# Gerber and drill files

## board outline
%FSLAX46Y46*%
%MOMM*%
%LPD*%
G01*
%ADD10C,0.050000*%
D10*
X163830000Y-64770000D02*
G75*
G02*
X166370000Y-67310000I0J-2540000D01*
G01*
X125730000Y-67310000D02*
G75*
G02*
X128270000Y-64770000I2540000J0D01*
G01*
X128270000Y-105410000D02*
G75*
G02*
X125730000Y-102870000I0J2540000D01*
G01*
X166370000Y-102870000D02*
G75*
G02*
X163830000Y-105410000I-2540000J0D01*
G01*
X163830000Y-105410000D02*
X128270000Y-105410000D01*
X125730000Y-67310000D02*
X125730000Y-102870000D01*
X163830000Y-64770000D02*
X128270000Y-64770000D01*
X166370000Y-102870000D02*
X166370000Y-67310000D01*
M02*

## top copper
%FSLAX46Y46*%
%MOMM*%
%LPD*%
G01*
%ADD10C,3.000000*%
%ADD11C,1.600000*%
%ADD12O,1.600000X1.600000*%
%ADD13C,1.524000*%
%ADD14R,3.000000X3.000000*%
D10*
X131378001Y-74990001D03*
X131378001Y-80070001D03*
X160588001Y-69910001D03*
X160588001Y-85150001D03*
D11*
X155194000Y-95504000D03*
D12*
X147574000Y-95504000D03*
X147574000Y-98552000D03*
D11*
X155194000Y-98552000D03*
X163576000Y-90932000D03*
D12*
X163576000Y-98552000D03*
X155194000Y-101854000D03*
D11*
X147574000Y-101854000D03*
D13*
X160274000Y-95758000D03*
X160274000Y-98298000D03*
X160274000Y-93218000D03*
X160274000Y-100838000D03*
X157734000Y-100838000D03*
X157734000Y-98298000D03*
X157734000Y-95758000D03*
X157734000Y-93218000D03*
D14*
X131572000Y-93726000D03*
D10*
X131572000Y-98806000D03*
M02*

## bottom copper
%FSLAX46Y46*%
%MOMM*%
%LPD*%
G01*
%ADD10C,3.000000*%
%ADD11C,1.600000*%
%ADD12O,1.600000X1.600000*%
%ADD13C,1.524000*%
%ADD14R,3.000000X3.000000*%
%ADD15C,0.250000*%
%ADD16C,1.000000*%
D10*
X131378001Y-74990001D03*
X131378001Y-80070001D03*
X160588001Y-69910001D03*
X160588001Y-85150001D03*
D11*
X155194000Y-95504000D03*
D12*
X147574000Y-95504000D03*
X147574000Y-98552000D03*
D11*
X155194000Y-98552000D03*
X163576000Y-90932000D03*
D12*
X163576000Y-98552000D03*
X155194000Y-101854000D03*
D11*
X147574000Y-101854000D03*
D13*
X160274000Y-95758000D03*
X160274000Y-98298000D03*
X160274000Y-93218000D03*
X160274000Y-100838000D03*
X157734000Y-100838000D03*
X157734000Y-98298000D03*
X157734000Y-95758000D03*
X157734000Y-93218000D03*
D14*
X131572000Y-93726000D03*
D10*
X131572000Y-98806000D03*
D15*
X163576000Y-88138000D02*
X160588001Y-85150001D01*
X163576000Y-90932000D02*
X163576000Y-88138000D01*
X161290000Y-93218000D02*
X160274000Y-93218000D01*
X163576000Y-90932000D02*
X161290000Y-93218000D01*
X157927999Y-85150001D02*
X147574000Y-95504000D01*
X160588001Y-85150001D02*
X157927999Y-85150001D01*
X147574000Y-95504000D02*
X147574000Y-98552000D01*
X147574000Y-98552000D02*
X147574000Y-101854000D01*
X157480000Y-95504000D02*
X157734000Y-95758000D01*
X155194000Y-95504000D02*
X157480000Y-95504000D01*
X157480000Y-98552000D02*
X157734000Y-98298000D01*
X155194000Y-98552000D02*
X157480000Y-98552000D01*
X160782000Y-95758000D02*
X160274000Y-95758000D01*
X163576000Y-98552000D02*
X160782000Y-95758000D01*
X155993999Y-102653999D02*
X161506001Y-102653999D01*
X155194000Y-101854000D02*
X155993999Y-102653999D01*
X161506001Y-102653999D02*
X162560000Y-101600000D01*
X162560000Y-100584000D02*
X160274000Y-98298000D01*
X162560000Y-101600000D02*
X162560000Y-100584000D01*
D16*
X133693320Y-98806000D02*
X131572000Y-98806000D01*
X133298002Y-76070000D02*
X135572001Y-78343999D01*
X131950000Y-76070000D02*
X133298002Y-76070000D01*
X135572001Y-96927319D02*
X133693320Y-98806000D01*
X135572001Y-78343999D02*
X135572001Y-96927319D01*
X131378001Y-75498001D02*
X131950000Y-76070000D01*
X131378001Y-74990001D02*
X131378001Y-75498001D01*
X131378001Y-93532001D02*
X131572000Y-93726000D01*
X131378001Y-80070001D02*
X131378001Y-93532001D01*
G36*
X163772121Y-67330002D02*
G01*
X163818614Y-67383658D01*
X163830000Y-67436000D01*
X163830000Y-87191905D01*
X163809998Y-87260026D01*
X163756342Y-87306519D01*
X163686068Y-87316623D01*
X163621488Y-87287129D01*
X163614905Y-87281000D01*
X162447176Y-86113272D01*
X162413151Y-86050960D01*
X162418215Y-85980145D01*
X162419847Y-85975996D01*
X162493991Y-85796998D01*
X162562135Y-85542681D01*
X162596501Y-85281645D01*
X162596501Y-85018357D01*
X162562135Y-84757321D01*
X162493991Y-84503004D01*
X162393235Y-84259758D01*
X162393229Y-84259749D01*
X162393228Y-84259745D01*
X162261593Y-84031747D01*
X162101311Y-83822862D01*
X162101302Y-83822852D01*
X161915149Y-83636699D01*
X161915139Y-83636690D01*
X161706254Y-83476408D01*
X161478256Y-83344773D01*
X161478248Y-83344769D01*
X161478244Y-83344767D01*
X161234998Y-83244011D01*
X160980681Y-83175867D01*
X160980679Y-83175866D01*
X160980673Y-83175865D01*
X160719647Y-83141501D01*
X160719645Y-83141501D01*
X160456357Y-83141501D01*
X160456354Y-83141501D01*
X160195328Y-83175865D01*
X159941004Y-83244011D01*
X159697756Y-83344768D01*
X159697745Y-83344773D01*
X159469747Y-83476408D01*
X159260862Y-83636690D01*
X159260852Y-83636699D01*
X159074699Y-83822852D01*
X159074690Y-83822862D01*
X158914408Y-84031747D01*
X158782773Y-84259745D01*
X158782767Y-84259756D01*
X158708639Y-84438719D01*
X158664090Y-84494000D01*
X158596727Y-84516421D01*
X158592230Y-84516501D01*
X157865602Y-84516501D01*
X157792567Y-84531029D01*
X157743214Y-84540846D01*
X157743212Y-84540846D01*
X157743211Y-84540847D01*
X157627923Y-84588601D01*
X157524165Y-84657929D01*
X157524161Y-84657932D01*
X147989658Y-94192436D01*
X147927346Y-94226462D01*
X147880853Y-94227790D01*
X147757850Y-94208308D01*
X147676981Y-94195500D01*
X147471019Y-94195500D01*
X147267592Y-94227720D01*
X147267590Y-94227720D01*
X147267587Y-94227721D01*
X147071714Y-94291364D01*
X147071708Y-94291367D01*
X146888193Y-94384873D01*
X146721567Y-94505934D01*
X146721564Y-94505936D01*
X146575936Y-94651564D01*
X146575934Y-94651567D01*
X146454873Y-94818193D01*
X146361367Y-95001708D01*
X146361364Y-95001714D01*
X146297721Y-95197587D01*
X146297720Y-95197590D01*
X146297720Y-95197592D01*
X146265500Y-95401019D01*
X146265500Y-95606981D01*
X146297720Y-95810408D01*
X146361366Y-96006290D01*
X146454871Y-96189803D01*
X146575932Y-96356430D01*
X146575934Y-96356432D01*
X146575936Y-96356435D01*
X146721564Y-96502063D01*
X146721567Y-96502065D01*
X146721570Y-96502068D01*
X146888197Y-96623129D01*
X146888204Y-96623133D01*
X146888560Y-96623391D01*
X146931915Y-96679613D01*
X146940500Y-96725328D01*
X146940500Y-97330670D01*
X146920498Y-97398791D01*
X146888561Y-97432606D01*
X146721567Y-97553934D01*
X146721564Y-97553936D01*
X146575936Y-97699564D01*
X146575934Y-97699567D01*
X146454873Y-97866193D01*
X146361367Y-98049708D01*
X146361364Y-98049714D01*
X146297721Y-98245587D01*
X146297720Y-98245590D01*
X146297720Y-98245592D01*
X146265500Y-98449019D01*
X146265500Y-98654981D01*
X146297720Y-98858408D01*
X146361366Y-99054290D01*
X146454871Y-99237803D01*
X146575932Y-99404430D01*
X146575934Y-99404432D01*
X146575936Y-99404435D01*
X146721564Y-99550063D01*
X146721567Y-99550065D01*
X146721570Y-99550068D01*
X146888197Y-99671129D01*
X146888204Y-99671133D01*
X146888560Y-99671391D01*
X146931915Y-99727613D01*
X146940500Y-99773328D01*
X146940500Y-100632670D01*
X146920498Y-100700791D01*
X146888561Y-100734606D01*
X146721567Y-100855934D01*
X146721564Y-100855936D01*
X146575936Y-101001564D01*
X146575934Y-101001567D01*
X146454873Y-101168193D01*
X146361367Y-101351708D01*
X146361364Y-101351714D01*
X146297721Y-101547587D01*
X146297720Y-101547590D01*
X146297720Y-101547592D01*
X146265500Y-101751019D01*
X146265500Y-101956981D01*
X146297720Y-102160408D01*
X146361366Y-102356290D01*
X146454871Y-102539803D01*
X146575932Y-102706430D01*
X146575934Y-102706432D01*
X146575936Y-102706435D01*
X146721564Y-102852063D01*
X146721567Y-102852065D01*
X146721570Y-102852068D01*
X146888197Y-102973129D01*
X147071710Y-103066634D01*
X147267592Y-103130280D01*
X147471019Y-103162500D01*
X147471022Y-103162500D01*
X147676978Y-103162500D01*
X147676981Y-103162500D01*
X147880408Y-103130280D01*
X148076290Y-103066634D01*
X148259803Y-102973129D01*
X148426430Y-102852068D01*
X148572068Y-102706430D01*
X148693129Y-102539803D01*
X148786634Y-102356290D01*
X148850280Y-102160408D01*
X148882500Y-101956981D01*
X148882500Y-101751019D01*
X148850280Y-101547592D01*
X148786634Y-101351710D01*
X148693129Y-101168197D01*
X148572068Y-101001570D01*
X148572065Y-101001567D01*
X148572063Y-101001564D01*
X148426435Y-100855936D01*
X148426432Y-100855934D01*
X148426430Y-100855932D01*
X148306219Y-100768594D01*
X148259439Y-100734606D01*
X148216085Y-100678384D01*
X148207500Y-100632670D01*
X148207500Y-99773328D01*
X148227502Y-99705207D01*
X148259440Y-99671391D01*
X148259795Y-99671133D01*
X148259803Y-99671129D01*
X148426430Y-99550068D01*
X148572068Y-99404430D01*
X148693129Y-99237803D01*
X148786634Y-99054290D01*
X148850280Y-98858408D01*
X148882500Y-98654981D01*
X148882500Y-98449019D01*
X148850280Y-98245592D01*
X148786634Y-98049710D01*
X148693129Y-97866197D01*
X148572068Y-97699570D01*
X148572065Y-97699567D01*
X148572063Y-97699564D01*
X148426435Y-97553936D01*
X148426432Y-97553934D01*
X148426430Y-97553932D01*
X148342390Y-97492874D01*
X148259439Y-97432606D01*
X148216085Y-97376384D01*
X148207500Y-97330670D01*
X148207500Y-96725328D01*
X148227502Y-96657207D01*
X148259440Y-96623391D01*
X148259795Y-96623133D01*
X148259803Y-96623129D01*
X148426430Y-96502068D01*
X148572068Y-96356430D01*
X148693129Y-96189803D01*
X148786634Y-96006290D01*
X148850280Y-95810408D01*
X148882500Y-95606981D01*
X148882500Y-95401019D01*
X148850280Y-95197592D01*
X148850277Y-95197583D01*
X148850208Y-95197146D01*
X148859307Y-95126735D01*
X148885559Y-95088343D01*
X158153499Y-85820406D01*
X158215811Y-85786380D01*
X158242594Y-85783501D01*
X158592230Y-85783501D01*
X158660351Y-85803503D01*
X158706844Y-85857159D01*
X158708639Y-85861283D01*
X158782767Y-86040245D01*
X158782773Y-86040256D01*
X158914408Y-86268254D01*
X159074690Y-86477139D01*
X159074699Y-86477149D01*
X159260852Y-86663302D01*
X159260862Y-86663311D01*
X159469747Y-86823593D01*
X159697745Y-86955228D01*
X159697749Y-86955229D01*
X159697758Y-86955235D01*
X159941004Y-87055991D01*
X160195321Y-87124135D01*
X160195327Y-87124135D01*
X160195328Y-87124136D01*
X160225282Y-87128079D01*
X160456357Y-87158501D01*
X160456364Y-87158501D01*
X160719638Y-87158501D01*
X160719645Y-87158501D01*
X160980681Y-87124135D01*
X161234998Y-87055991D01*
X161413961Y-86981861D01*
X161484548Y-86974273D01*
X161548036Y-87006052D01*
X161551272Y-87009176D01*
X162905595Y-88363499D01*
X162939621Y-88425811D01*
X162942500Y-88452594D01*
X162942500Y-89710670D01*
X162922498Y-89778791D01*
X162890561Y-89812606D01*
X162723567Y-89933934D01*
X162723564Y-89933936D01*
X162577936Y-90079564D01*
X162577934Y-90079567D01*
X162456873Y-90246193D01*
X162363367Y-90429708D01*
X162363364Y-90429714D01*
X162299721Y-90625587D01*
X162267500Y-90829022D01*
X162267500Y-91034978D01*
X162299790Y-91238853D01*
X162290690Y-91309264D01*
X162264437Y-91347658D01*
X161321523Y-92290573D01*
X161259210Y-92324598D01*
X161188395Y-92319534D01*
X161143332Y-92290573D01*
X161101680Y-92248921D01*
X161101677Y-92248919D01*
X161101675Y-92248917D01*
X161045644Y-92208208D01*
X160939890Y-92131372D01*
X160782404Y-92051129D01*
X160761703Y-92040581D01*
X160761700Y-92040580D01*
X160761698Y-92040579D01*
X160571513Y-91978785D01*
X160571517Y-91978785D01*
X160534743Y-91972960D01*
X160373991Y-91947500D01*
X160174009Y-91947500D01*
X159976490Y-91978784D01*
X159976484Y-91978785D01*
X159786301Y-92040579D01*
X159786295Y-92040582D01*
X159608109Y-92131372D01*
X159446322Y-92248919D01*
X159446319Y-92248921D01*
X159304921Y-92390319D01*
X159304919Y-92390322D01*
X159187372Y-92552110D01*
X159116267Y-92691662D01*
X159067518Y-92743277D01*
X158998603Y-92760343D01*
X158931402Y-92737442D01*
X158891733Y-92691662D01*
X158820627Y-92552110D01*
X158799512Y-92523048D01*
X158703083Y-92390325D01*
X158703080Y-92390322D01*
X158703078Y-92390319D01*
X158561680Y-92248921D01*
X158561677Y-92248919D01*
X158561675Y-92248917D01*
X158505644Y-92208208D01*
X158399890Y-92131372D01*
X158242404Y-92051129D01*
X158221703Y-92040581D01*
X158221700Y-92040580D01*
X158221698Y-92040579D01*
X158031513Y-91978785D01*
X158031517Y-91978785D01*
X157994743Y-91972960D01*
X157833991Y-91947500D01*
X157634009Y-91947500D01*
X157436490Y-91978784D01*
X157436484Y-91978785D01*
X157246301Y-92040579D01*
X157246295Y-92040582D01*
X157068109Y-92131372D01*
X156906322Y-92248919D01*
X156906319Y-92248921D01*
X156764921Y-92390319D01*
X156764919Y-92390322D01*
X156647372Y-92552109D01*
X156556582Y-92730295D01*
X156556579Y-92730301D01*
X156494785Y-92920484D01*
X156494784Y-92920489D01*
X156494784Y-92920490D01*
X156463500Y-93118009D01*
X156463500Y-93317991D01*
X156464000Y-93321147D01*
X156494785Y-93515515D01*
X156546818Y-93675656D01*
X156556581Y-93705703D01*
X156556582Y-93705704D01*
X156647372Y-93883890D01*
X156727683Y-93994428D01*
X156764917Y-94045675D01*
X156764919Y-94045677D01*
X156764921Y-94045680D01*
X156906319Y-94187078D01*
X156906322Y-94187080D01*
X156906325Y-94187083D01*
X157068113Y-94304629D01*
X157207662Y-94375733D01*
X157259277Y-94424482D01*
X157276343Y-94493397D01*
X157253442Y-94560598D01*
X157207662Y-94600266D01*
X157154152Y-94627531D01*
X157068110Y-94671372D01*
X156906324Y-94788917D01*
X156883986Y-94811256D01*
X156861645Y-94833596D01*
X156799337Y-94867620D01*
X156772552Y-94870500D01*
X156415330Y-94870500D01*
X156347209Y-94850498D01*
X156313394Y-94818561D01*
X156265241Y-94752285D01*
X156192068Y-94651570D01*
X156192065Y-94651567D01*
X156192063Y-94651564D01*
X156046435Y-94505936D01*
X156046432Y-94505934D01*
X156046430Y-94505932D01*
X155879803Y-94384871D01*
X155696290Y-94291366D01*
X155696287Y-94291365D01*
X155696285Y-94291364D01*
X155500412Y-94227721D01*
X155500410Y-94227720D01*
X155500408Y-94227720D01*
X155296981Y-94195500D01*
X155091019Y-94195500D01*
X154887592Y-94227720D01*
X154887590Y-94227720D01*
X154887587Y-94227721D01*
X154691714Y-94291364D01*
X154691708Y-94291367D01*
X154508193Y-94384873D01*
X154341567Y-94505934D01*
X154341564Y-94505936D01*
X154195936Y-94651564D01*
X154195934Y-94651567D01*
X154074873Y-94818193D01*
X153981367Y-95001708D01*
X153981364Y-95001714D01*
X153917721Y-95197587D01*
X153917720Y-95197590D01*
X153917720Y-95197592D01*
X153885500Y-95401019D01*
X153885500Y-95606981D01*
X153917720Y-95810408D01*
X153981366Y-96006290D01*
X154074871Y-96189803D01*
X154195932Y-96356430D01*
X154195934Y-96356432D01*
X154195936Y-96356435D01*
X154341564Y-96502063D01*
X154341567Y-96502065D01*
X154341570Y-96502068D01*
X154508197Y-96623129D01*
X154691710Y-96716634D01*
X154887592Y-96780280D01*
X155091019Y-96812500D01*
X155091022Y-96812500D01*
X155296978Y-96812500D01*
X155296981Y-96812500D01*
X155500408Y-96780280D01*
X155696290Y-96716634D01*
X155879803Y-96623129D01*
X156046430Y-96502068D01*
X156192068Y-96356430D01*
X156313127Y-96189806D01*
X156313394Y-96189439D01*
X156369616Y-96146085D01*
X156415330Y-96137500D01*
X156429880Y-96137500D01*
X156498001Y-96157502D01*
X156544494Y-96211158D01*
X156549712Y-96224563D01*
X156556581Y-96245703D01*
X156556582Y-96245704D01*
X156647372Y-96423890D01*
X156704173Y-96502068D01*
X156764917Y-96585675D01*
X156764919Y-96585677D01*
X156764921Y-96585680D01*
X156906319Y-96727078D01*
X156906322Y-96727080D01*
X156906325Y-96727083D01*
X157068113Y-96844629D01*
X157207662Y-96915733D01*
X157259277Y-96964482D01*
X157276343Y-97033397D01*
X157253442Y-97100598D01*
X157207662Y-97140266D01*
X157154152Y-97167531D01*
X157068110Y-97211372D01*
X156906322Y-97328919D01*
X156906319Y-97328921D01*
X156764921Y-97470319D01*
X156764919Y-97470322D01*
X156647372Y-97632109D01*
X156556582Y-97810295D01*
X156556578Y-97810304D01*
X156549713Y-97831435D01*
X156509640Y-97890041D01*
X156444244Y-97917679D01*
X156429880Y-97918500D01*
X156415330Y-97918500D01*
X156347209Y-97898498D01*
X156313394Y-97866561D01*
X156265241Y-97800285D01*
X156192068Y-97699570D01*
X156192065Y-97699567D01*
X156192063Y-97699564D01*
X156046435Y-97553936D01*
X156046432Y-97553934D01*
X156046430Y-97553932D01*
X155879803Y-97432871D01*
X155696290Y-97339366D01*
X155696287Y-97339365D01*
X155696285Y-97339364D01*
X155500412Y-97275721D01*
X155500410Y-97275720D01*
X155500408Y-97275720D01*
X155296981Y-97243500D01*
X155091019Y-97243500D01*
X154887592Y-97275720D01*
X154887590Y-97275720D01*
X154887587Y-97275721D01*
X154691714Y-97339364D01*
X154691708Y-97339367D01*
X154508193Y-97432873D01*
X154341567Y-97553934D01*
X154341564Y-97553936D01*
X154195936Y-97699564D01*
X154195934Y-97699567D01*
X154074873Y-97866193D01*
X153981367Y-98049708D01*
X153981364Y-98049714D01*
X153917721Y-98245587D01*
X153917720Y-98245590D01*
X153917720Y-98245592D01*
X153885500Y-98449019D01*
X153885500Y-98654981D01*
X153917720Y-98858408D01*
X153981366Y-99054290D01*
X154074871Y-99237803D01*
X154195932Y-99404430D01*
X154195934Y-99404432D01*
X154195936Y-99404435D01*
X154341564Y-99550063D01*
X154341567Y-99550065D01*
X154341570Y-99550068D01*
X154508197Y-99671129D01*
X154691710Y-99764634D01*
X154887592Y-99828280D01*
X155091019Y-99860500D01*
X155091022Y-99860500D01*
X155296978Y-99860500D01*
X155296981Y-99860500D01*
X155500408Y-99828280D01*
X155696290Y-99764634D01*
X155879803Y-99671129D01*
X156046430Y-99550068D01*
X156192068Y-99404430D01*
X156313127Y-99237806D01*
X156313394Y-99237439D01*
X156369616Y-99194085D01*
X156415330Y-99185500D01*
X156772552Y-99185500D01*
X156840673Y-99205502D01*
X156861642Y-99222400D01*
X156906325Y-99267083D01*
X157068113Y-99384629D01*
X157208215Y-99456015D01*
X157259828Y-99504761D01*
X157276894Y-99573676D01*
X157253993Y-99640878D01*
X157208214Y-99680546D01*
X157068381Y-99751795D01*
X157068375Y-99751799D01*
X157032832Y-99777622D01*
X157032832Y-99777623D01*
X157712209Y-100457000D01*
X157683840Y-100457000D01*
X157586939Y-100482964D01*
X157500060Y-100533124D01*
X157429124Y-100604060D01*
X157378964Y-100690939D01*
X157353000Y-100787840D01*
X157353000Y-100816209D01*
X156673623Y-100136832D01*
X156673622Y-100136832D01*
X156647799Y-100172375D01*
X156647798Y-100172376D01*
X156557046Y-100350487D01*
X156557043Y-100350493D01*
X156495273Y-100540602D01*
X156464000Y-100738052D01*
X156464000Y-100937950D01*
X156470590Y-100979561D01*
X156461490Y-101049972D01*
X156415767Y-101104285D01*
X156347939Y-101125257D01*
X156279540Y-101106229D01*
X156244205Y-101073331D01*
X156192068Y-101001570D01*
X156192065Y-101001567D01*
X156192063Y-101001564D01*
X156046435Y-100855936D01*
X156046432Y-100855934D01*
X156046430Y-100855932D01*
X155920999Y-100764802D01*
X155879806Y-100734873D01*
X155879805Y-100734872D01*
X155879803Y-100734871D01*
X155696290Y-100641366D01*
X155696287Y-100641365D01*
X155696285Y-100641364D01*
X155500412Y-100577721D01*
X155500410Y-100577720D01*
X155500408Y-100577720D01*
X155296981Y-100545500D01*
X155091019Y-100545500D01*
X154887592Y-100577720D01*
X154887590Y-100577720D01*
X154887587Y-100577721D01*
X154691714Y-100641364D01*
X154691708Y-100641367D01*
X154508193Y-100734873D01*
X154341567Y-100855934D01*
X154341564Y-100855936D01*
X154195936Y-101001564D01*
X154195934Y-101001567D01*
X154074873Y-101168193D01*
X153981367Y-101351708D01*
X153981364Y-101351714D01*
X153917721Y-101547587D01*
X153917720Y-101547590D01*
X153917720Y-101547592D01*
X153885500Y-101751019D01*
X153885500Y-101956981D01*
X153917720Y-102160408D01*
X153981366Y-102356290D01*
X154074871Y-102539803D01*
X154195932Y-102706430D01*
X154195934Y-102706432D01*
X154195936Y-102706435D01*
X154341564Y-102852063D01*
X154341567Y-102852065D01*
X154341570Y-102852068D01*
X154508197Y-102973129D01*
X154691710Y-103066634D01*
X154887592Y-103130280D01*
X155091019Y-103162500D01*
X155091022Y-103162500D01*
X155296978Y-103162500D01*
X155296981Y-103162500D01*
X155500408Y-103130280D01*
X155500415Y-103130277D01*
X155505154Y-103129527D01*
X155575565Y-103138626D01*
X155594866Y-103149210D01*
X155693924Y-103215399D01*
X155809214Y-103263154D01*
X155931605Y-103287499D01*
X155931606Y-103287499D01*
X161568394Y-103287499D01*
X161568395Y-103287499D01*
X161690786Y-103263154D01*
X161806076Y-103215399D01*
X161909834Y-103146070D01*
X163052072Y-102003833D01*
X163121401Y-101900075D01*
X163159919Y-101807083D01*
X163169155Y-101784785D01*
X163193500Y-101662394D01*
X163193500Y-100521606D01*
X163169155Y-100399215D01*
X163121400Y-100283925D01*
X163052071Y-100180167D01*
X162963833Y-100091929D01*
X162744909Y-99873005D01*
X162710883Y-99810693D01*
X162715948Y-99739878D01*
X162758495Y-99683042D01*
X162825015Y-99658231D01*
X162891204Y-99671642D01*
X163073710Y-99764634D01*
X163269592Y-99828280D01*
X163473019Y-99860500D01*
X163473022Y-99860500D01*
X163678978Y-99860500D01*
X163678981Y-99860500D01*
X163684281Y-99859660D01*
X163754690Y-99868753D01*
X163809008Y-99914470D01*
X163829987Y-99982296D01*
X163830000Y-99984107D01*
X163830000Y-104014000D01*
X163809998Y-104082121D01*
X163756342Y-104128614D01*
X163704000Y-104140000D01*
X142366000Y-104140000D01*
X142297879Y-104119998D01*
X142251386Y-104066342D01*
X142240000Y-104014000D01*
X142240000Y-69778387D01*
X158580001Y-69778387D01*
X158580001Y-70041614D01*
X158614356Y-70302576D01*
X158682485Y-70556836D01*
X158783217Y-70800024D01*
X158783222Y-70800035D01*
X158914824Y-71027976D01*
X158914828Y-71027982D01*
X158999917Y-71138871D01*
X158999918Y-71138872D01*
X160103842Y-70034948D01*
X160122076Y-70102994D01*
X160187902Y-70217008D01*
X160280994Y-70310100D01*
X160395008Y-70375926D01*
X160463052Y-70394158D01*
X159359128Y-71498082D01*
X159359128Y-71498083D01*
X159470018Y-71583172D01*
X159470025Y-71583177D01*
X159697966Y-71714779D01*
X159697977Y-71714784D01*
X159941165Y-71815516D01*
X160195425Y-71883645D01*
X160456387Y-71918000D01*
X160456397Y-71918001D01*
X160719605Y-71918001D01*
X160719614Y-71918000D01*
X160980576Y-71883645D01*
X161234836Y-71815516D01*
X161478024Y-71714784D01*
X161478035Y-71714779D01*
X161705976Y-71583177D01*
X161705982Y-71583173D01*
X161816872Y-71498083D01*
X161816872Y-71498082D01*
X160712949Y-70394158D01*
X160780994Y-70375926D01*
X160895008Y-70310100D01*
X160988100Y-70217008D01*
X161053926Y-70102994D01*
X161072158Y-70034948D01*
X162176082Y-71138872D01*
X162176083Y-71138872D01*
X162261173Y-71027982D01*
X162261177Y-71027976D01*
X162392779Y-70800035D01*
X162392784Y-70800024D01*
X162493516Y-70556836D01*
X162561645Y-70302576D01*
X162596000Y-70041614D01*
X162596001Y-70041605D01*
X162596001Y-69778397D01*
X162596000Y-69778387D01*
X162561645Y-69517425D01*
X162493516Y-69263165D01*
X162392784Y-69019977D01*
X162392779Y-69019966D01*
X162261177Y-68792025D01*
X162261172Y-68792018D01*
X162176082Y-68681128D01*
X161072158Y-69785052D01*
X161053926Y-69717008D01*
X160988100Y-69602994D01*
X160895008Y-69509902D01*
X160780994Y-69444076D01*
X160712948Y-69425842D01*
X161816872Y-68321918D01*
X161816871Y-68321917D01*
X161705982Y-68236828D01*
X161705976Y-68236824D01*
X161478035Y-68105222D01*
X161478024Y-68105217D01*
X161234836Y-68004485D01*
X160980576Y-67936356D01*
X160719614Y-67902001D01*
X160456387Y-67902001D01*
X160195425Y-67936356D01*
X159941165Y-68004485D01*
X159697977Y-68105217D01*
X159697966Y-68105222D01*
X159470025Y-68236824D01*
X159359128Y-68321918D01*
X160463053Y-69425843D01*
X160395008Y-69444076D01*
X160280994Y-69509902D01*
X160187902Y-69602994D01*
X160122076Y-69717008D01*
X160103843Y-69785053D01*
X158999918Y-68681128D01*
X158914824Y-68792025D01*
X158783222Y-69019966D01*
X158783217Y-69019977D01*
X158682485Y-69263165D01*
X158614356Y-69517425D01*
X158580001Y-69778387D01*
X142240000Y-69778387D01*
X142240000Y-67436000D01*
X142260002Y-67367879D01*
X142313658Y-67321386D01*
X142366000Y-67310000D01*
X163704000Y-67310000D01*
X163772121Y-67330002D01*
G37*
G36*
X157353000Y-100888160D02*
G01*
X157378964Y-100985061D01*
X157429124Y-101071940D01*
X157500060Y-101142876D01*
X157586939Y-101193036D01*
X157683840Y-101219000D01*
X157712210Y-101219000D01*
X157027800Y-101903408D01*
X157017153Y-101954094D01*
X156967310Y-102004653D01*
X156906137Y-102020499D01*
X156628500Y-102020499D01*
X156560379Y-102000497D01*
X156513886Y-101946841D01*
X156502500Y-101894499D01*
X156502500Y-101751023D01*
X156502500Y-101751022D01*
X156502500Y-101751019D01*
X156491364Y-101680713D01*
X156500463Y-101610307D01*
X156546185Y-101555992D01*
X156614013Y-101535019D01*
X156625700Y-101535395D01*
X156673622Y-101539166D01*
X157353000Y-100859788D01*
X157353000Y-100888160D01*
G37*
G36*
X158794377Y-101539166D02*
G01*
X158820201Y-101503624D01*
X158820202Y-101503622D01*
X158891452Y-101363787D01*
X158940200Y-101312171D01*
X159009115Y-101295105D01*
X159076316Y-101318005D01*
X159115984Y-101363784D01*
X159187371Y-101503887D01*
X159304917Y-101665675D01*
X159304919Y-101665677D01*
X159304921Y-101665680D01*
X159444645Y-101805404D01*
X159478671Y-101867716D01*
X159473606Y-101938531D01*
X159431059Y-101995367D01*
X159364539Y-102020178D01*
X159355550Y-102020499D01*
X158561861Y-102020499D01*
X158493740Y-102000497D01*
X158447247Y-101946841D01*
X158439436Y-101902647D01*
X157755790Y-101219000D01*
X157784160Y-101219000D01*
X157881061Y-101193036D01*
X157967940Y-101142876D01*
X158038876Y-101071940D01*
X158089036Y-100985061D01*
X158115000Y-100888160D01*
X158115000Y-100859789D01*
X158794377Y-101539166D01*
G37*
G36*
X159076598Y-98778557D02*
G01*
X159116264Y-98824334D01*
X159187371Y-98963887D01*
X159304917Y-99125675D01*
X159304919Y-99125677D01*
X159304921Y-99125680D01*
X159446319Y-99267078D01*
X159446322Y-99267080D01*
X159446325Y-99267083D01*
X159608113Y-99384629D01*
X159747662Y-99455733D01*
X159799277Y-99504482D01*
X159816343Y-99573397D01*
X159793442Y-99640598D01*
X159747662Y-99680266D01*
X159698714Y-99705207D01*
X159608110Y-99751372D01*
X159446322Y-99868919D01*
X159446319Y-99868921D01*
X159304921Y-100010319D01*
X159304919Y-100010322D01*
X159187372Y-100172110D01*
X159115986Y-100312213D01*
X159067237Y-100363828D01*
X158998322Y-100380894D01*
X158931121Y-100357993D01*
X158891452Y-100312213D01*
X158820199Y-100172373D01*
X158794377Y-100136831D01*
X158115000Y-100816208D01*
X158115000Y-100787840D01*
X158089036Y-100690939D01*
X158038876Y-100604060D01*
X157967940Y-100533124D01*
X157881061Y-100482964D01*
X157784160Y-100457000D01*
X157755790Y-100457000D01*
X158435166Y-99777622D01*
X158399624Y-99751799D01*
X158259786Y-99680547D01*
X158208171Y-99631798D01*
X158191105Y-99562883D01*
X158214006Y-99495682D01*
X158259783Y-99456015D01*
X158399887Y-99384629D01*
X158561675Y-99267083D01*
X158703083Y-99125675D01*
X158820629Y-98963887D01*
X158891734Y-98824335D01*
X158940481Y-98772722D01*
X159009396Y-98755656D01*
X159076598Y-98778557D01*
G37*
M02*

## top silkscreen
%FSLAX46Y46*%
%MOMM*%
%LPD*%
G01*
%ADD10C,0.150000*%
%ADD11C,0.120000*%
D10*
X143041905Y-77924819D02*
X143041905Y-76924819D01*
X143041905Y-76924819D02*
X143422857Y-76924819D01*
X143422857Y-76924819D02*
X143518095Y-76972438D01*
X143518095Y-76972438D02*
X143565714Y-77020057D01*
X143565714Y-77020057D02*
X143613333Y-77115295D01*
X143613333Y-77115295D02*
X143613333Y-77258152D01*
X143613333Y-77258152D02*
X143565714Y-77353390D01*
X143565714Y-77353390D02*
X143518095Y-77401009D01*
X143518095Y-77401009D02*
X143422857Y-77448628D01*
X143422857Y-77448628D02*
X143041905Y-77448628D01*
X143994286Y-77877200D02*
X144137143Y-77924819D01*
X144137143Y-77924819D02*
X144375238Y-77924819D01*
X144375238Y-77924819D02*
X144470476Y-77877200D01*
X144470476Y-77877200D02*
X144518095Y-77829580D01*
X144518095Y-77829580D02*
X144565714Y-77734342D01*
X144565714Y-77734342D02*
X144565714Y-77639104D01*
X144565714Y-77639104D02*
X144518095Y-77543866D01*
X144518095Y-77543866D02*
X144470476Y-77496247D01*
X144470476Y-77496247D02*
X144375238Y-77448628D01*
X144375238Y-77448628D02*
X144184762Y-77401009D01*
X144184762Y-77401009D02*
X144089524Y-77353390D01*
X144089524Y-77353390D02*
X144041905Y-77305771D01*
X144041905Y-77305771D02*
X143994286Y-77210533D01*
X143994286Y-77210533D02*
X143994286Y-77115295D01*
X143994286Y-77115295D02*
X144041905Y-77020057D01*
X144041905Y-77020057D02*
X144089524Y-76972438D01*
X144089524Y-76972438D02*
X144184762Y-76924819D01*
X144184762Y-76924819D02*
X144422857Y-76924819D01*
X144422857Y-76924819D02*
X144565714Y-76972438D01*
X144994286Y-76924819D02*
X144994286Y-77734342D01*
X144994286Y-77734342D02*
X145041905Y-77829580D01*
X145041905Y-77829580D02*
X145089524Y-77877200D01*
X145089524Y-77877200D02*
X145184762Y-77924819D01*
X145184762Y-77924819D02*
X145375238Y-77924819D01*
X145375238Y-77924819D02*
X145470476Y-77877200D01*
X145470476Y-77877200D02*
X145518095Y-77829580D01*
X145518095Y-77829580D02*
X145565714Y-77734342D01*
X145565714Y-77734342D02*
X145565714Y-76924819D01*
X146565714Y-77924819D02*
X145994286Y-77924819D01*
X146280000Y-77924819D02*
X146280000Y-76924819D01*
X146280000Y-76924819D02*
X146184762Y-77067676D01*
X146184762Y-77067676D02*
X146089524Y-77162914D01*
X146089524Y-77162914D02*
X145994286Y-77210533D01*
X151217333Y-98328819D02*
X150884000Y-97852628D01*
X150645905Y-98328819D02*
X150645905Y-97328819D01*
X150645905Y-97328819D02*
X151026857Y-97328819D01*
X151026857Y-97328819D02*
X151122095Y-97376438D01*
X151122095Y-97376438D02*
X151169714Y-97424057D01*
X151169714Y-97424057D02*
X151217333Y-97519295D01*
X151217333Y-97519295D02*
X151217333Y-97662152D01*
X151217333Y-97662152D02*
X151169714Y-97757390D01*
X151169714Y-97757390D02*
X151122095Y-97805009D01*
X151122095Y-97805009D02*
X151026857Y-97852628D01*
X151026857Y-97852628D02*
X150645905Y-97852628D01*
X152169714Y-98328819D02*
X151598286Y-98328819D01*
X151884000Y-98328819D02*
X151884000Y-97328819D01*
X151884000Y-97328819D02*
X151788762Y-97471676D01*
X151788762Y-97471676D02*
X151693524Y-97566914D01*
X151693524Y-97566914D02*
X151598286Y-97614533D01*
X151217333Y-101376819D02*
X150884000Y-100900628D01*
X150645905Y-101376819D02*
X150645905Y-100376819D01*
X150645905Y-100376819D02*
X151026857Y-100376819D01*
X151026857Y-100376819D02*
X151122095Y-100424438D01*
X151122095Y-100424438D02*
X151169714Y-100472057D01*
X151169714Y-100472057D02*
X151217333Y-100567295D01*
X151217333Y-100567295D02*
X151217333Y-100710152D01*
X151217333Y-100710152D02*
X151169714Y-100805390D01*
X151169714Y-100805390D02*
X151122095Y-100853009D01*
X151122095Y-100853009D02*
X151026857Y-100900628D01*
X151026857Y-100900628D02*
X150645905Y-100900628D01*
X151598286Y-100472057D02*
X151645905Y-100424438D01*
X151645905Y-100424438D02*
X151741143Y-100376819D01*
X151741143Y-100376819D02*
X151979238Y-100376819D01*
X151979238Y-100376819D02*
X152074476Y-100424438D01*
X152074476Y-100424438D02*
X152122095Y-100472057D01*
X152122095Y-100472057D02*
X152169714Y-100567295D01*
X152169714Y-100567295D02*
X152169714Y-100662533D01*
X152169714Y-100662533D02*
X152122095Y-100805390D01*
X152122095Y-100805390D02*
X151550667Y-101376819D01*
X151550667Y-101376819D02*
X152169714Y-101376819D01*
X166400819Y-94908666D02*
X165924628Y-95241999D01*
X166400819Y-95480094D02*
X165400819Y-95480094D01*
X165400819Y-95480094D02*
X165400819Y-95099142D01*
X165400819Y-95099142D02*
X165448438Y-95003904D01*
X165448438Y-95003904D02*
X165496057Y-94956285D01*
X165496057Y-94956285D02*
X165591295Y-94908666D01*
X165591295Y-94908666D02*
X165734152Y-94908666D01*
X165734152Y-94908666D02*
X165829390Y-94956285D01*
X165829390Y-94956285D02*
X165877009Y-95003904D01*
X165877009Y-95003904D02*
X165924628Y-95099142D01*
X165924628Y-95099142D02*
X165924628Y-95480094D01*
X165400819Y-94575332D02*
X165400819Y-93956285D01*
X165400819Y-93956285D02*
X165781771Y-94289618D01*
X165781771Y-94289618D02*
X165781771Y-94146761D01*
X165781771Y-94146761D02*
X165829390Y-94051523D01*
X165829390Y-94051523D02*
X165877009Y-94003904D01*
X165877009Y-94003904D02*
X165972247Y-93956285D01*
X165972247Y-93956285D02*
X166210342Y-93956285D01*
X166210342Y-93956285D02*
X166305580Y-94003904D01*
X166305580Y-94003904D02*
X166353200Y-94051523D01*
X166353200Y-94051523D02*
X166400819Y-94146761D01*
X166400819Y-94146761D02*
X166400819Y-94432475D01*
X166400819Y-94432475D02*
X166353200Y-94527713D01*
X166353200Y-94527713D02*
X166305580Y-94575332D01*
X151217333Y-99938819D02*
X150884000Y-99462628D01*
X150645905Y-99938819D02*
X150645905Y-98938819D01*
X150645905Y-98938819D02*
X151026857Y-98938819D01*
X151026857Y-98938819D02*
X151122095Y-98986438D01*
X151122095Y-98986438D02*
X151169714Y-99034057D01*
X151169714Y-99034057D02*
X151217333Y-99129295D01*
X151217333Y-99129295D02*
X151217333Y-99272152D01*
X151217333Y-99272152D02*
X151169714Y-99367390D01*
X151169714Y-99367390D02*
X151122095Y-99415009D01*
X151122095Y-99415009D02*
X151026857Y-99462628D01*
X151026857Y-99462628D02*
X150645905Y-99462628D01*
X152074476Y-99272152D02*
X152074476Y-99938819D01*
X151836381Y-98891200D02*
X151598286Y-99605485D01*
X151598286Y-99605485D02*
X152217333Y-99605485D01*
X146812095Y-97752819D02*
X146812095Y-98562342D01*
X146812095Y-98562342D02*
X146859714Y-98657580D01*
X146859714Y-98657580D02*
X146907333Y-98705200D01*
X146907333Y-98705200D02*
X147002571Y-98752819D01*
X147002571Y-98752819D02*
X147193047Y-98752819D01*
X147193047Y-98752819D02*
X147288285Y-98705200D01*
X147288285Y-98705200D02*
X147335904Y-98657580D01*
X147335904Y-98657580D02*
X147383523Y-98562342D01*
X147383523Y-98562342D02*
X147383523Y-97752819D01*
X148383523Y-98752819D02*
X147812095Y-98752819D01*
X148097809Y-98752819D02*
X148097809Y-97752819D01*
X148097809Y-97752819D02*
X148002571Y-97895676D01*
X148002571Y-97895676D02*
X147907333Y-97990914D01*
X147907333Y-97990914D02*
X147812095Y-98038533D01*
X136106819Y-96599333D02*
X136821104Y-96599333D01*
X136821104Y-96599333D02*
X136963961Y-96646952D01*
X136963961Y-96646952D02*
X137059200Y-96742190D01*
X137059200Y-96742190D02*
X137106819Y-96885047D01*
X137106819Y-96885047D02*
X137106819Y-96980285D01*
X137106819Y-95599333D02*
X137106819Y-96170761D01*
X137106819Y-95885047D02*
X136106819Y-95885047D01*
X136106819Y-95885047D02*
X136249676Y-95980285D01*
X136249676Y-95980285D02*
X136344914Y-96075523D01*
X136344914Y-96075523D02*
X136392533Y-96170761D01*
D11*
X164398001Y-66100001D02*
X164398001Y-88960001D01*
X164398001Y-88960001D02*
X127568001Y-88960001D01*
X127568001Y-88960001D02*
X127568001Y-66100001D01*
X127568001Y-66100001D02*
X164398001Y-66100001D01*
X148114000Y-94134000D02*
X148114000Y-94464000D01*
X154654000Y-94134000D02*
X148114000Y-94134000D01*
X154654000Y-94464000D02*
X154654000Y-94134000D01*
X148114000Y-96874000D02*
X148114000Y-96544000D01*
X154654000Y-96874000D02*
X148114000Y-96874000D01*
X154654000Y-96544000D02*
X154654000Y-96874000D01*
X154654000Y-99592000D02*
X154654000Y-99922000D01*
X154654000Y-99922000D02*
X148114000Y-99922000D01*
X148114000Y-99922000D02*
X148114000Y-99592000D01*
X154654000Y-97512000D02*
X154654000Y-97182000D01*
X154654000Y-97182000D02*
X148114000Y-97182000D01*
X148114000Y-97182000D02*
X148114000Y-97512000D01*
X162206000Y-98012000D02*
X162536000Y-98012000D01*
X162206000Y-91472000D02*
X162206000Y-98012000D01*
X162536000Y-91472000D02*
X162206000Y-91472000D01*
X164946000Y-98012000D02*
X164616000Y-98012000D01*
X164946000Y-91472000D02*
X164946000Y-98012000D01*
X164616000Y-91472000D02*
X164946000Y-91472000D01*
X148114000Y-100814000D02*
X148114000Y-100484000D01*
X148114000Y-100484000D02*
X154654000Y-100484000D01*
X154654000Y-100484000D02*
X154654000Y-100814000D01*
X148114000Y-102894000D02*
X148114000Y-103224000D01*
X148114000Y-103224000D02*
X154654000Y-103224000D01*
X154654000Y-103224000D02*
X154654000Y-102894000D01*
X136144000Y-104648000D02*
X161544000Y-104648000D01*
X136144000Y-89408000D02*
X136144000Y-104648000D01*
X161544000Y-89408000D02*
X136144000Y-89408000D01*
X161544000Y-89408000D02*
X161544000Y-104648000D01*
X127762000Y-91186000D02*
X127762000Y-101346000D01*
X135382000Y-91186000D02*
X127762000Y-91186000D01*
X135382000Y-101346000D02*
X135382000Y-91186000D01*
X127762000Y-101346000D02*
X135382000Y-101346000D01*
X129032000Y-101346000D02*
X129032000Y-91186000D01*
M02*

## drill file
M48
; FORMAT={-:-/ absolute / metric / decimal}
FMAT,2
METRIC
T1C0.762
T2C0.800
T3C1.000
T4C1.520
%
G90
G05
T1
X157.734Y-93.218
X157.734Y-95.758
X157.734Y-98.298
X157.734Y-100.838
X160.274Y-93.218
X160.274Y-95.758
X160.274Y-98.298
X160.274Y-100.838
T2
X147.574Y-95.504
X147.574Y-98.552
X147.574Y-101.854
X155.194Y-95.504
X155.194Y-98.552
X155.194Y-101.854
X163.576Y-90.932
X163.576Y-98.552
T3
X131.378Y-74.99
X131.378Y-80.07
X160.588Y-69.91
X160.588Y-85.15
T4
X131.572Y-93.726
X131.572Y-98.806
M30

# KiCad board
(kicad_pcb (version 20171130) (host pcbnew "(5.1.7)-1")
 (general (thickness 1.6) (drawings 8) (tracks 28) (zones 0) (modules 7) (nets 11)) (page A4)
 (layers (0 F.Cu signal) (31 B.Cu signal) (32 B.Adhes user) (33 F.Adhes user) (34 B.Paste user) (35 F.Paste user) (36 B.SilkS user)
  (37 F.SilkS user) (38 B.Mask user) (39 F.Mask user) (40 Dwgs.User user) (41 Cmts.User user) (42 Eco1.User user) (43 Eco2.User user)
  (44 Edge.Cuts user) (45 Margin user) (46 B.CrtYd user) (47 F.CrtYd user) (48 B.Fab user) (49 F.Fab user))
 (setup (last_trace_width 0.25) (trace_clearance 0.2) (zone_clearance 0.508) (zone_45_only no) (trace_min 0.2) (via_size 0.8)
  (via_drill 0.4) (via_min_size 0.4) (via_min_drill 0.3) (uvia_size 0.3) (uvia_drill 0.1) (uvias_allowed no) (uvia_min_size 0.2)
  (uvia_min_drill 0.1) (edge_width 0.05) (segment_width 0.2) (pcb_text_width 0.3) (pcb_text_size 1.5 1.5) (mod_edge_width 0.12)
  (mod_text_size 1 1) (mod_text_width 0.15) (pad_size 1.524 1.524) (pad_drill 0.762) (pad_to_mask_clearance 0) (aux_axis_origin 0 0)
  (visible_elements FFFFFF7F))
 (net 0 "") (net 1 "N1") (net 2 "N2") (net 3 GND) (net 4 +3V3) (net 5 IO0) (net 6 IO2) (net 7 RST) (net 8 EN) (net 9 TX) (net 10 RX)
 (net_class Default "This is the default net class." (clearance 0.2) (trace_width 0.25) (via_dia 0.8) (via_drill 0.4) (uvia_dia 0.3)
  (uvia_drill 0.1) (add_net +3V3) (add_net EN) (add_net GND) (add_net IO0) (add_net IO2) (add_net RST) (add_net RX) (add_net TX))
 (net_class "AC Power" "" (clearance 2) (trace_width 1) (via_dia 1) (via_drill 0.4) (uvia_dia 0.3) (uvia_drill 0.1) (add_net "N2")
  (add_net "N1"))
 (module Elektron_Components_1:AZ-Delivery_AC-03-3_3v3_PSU (layer F.Cu) (at 146.618001 77.530001)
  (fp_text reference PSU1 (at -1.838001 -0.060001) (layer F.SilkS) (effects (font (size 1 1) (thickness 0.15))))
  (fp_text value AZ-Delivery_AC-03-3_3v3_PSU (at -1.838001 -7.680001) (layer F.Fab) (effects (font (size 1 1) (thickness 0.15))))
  (fp_line (start 17.78 -11.43) (end 17.78 11.43) (layer F.SilkS) (width 0.12))
  (fp_line (start 17.78 11.43) (end -19.05 11.43) (layer F.SilkS) (width 0.12))
  (fp_line (start -19.05 11.43) (end -19.05 -11.43) (layer F.SilkS) (width 0.12))
  (fp_line (start -19.05 -11.43) (end 17.78 -11.43) (layer F.SilkS) (width 0.12))
  (pad 1 thru_hole circle (at -15.24 -2.54) (size 3 3) (drill 1) (layers *.Cu *.Mask) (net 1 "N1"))
  (pad 2 thru_hole circle (at -15.24 2.54) (size 3 3) (drill 1) (layers *.Cu *.Mask) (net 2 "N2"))
  (pad 3 thru_hole circle (at 13.97 -7.62) (size 3 3) (drill 1) (layers *.Cu *.Mask) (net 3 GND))
  (pad 4 thru_hole circle (at 13.97 7.62) (size 3 3) (drill 1) (layers *.Cu *.Mask) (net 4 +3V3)))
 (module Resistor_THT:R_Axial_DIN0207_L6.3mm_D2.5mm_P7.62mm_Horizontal (layer F.Cu) (at 155.194 95.504 180)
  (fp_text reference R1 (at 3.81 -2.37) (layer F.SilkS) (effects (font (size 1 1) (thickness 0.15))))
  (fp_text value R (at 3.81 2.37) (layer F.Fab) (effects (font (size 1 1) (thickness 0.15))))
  (fp_line (start 7.08 1.37) (end 7.08 1.04) (layer F.SilkS) (width 0.12))
  (fp_line (start 0.54 1.37) (end 7.08 1.37) (layer F.SilkS) (width 0.12))
  (fp_line (start 0.54 1.04) (end 0.54 1.37) (layer F.SilkS) (width 0.12))
  (fp_line (start 7.08 -1.37) (end 7.08 -1.04) (layer F.SilkS) (width 0.12))
  (fp_line (start 0.54 -1.37) (end 7.08 -1.37) (layer F.SilkS) (width 0.12))
  (fp_line (start 0.54 -1.04) (end 0.54 -1.37) (layer F.SilkS) (width 0.12))
  (pad 1 thru_hole circle (at 0 0 180) (size 1.6 1.6) (drill 0.8) (layers *.Cu *.Mask) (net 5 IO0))
  (pad 2 thru_hole oval (at 7.62 0 180) (size 1.6 1.6) (drill 0.8) (layers *.Cu *.Mask) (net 4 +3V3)))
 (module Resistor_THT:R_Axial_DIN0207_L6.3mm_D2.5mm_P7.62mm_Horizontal (layer F.Cu) (at 155.194 98.552 180)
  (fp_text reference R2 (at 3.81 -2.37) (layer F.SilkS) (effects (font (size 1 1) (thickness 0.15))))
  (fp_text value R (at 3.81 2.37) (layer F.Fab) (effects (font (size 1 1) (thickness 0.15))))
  (fp_line (start 0.54 -1.04) (end 0.54 -1.37) (layer F.SilkS) (width 0.12))
  (fp_line (start 0.54 -1.37) (end 7.08 -1.37) (layer F.SilkS) (width 0.12))
  (fp_line (start 7.08 -1.37) (end 7.08 -1.04) (layer F.SilkS) (width 0.12))
  (fp_line (start 0.54 1.04) (end 0.54 1.37) (layer F.SilkS) (width 0.12))
  (fp_line (start 0.54 1.37) (end 7.08 1.37) (layer F.SilkS) (width 0.12))
  (fp_line (start 7.08 1.37) (end 7.08 1.04) (layer F.SilkS) (width 0.12))
  (pad 2 thru_hole oval (at 7.62 0 180) (size 1.6 1.6) (drill 0.8) (layers *.Cu *.Mask) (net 4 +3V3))
  (pad 1 thru_hole circle (at 0 0 180) (size 1.6 1.6) (drill 0.8) (layers *.Cu *.Mask) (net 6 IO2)))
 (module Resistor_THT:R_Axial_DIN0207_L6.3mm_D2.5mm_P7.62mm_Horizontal (layer F.Cu) (at 163.576 90.932 270)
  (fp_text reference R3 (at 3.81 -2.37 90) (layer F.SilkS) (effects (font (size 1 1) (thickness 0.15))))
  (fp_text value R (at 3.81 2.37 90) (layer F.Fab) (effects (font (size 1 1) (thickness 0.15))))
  (fp_line (start 7.08 1.37) (end 7.08 1.04) (layer F.SilkS) (width 0.12))
  (fp_line (start 0.54 1.37) (end 7.08 1.37) (layer F.SilkS) (width 0.12))
  (fp_line (start 0.54 1.04) (end 0.54 1.37) (layer F.SilkS) (width 0.12))
  (fp_line (start 7.08 -1.37) (end 7.08 -1.04) (layer F.SilkS) (width 0.12))
  (fp_line (start 0.54 -1.37) (end 7.08 -1.37) (layer F.SilkS) (width 0.12))
  (fp_line (start 0.54 -1.04) (end 0.54 -1.37) (layer F.SilkS) (width 0.12))
  (pad 1 thru_hole circle (at 0 0 270) (size 1.6 1.6) (drill 0.8) (layers *.Cu *.Mask) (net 4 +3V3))
  (pad 2 thru_hole oval (at 7.62 0 270) (size 1.6 1.6) (drill 0.8) (layers *.Cu *.Mask) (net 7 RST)))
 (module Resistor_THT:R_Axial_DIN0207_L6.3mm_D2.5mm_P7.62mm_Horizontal (layer F.Cu) (at 147.574 101.854)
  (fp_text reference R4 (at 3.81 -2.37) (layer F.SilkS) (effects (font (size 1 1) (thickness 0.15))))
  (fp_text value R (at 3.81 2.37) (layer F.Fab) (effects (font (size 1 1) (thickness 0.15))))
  (fp_line (start 0.54 -1.04) (end 0.54 -1.37) (layer F.SilkS) (width 0.12))
  (fp_line (start 0.54 -1.37) (end 7.08 -1.37) (layer F.SilkS) (width 0.12))
  (fp_line (start 7.08 -1.37) (end 7.08 -1.04) (layer F.SilkS) (width 0.12))
  (fp_line (start 0.54 1.04) (end 0.54 1.37) (layer F.SilkS) (width 0.12))
  (fp_line (start 0.54 1.37) (end 7.08 1.37) (layer F.SilkS) (width 0.12))
  (fp_line (start 7.08 1.37) (end 7.08 1.04) (layer F.SilkS) (width 0.12))
  (pad 2 thru_hole oval (at 7.62 0) (size 1.6 1.6) (drill 0.8) (layers *.Cu *.Mask) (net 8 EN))
  (pad 1 thru_hole circle (at 0 0) (size 1.6 1.6) (drill 0.8) (layers *.Cu *.Mask) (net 4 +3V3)))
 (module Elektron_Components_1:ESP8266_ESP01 (layer F.Cu) (at 159.004 97.028)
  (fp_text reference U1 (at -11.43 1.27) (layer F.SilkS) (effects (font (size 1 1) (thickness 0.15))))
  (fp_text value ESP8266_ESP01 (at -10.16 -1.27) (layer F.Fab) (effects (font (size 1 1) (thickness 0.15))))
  (fp_line (start -22.86 7.62) (end 2.54 7.62) (layer F.SilkS) (width 0.12))
  (fp_line (start -22.86 -7.62) (end -22.86 7.62) (layer F.SilkS) (width 0.12))
  (fp_line (start 2.54 -7.62) (end -22.86 -7.62) (layer F.SilkS) (width 0.12))
  (fp_line (start 2.54 -7.62) (end 2.54 7.62) (layer F.SilkS) (width 0.12))
  (pad 3 thru_hole circle (at 1.27 -1.27) (size 1.524 1.524) (drill 0.762) (layers *.Cu *.Mask) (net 7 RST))
  (pad 2 thru_hole circle (at 1.27 1.27) (size 1.524 1.524) (drill 0.762) (layers *.Cu *.Mask) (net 8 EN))
  (pad 4 thru_hole circle (at 1.27 -3.81) (size 1.524 1.524) (drill 0.762) (layers *.Cu *.Mask) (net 4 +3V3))
  (pad 1 thru_hole circle (at 1.27 3.81) (size 1.524 1.524) (drill 0.762) (layers *.Cu *.Mask) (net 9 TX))
  (pad 5 thru_hole circle (at -1.27 3.81) (size 1.524 1.524) (drill 0.762) (layers *.Cu *.Mask) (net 3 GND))
  (pad 6 thru_hole circle (at -1.27 1.27) (size 1.524 1.524) (drill 0.762) (layers *.Cu *.Mask) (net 6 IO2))
  (pad 7 thru_hole circle (at -1.27 -1.27) (size 1.524 1.524) (drill 0.762) (layers *.Cu *.Mask) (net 5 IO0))
  (pad 8 thru_hole circle (at -1.27 -3.81) (size 1.524 1.524) (drill 0.762) (layers *.Cu *.Mask) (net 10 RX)))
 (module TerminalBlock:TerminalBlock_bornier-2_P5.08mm (layer F.Cu) (at 131.572 93.726 270)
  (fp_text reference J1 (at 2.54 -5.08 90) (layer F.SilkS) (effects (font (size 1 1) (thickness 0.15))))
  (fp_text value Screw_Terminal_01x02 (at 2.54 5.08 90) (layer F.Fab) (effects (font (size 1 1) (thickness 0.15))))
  (fp_line (start -2.54 3.81) (end 7.62 3.81) (layer F.SilkS) (width 0.12))
  (fp_line (start -2.54 -3.81) (end -2.54 3.81) (layer F.SilkS) (width 0.12))
  (fp_line (start 7.62 -3.81) (end -2.54 -3.81) (layer F.SilkS) (width 0.12))
  (fp_line (start 7.62 3.81) (end 7.62 -3.81) (layer F.SilkS) (width 0.12))
  (fp_line (start 7.62 2.54) (end -2.54 2.54) (layer F.SilkS) (width 0.12))
  (pad 1 thru_hole rect (at 0 0 270) (size 3 3) (drill 1.52) (layers *.Cu *.Mask) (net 2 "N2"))
  (pad 2 thru_hole circle (at 5.08 0 270) (size 3 3) (drill 1.52) (layers *.Cu *.Mask) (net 1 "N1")))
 (gr_arc (start 163.83 67.31) (end 166.37 67.31) (angle -90) (layer Edge.Cuts) (width 0.05))
 (gr_arc (start 128.27 67.31) (end 128.27 64.77) (angle -90) (layer Edge.Cuts) (width 0.05))
 (gr_arc (start 128.27 102.87) (end 125.73 102.87) (angle -90) (layer Edge.Cuts) (width 0.05))
 (gr_arc (start 163.83 102.87) (end 163.83 105.41) (angle -90) (layer Edge.Cuts) (width 0.05))
 (gr_line (start 163.83 105.41) (end 128.27 105.41) (layer Edge.Cuts) (width 0.05))
 (gr_line (start 125.73 67.31) (end 125.73 102.87) (layer Edge.Cuts) (width 0.05))
 (gr_line (start 163.83 64.77) (end 128.27 64.77) (layer Edge.Cuts) (width 0.05))
 (gr_line (start 166.37 102.87) (end 166.37 67.31) (layer Edge.Cuts) (width 0.05))
 (segment (start 163.576 88.138) (end 160.588001 85.150001) (width 0.25) (layer B.Cu) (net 4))
 (segment (start 163.576 90.932) (end 163.576 88.138) (width 0.25) (layer B.Cu) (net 4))
 (segment (start 161.29 93.218) (end 160.274 93.218) (width 0.25) (layer B.Cu) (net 4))
 (segment (start 163.576 90.932) (end 161.29 93.218) (width 0.25) (layer B.Cu) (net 4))
 (segment (start 157.927999 85.150001) (end 147.574 95.504) (width 0.25) (layer B.Cu) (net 4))
 (segment (start 160.588001 85.150001) (end 157.927999 85.150001) (width 0.25) (layer B.Cu) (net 4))
 (segment (start 147.574 95.504) (end 147.574 98.552) (width 0.25) (layer B.Cu) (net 4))
 (segment (start 147.574 98.552) (end 147.574 101.854) (width 0.25) (layer B.Cu) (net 4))
 (segment (start 157.48 95.504) (end 157.734 95.758) (width 0.25) (layer B.Cu) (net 5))
 (segment (start 155.194 95.504) (end 157.48 95.504) (width 0.25) (layer B.Cu) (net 5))
 (segment (start 157.48 98.552) (end 157.734 98.298) (width 0.25) (layer B.Cu) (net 6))
 (segment (start 155.194 98.552) (end 157.48 98.552) (width 0.25) (layer B.Cu) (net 6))
 (segment (start 160.782 95.758) (end 160.274 95.758) (width 0.25) (layer B.Cu) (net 7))
 (segment (start 163.576 98.552) (end 160.782 95.758) (width 0.25) (layer B.Cu) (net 7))
 (segment (start 155.993999 102.653999) (end 161.506001 102.653999) (width 0.25) (layer B.Cu) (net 8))
 (segment (start 155.194 101.854) (end 155.993999 102.653999) (width 0.25) (layer B.Cu) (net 8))
 (segment (start 161.506001 102.653999) (end 162.56 101.6) (width 0.25) (layer B.Cu) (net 8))
 (segment (start 162.56 100.584) (end 160.274 98.298) (width 0.25) (layer B.Cu) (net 8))
 (segment (start 162.56 101.6) (end 162.56 100.584) (width 0.25) (layer B.Cu) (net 8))
 (segment (start 133.69332 98.806) (end 131.572 98.806) (width 1) (layer B.Cu) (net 1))
 (segment (start 133.298002 76.07) (end 135.572001 78.343999) (width 1) (layer B.Cu) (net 1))
 (segment (start 131.95 76.07) (end 133.298002 76.07) (width 1) (layer B.Cu) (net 1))
 (segment (start 135.572001 96.927319) (end 133.69332 98.806) (width 1) (layer B.Cu) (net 1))
 (segment (start 135.572001 78.343999) (end 135.572001 96.927319) (width 1) (layer B.Cu) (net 1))
 (segment (start 131.378001 75.498001) (end 131.95 76.07) (width 1) (layer B.Cu) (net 1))
 (segment (start 131.378001 74.990001) (end 131.378001 75.498001) (width 1) (layer B.Cu) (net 1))
 (segment (start 131.378001 93.532001) (end 131.572 93.726) (width 1) (layer B.Cu) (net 2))
 (segment (start 131.378001 80.070001) (end 131.378001 93.532001) (width 1) (layer B.Cu) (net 2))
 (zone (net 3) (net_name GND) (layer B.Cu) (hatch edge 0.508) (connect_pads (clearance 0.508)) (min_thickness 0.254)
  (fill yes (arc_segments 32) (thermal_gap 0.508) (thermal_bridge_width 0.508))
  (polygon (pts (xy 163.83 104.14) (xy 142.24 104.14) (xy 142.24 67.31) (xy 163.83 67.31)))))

